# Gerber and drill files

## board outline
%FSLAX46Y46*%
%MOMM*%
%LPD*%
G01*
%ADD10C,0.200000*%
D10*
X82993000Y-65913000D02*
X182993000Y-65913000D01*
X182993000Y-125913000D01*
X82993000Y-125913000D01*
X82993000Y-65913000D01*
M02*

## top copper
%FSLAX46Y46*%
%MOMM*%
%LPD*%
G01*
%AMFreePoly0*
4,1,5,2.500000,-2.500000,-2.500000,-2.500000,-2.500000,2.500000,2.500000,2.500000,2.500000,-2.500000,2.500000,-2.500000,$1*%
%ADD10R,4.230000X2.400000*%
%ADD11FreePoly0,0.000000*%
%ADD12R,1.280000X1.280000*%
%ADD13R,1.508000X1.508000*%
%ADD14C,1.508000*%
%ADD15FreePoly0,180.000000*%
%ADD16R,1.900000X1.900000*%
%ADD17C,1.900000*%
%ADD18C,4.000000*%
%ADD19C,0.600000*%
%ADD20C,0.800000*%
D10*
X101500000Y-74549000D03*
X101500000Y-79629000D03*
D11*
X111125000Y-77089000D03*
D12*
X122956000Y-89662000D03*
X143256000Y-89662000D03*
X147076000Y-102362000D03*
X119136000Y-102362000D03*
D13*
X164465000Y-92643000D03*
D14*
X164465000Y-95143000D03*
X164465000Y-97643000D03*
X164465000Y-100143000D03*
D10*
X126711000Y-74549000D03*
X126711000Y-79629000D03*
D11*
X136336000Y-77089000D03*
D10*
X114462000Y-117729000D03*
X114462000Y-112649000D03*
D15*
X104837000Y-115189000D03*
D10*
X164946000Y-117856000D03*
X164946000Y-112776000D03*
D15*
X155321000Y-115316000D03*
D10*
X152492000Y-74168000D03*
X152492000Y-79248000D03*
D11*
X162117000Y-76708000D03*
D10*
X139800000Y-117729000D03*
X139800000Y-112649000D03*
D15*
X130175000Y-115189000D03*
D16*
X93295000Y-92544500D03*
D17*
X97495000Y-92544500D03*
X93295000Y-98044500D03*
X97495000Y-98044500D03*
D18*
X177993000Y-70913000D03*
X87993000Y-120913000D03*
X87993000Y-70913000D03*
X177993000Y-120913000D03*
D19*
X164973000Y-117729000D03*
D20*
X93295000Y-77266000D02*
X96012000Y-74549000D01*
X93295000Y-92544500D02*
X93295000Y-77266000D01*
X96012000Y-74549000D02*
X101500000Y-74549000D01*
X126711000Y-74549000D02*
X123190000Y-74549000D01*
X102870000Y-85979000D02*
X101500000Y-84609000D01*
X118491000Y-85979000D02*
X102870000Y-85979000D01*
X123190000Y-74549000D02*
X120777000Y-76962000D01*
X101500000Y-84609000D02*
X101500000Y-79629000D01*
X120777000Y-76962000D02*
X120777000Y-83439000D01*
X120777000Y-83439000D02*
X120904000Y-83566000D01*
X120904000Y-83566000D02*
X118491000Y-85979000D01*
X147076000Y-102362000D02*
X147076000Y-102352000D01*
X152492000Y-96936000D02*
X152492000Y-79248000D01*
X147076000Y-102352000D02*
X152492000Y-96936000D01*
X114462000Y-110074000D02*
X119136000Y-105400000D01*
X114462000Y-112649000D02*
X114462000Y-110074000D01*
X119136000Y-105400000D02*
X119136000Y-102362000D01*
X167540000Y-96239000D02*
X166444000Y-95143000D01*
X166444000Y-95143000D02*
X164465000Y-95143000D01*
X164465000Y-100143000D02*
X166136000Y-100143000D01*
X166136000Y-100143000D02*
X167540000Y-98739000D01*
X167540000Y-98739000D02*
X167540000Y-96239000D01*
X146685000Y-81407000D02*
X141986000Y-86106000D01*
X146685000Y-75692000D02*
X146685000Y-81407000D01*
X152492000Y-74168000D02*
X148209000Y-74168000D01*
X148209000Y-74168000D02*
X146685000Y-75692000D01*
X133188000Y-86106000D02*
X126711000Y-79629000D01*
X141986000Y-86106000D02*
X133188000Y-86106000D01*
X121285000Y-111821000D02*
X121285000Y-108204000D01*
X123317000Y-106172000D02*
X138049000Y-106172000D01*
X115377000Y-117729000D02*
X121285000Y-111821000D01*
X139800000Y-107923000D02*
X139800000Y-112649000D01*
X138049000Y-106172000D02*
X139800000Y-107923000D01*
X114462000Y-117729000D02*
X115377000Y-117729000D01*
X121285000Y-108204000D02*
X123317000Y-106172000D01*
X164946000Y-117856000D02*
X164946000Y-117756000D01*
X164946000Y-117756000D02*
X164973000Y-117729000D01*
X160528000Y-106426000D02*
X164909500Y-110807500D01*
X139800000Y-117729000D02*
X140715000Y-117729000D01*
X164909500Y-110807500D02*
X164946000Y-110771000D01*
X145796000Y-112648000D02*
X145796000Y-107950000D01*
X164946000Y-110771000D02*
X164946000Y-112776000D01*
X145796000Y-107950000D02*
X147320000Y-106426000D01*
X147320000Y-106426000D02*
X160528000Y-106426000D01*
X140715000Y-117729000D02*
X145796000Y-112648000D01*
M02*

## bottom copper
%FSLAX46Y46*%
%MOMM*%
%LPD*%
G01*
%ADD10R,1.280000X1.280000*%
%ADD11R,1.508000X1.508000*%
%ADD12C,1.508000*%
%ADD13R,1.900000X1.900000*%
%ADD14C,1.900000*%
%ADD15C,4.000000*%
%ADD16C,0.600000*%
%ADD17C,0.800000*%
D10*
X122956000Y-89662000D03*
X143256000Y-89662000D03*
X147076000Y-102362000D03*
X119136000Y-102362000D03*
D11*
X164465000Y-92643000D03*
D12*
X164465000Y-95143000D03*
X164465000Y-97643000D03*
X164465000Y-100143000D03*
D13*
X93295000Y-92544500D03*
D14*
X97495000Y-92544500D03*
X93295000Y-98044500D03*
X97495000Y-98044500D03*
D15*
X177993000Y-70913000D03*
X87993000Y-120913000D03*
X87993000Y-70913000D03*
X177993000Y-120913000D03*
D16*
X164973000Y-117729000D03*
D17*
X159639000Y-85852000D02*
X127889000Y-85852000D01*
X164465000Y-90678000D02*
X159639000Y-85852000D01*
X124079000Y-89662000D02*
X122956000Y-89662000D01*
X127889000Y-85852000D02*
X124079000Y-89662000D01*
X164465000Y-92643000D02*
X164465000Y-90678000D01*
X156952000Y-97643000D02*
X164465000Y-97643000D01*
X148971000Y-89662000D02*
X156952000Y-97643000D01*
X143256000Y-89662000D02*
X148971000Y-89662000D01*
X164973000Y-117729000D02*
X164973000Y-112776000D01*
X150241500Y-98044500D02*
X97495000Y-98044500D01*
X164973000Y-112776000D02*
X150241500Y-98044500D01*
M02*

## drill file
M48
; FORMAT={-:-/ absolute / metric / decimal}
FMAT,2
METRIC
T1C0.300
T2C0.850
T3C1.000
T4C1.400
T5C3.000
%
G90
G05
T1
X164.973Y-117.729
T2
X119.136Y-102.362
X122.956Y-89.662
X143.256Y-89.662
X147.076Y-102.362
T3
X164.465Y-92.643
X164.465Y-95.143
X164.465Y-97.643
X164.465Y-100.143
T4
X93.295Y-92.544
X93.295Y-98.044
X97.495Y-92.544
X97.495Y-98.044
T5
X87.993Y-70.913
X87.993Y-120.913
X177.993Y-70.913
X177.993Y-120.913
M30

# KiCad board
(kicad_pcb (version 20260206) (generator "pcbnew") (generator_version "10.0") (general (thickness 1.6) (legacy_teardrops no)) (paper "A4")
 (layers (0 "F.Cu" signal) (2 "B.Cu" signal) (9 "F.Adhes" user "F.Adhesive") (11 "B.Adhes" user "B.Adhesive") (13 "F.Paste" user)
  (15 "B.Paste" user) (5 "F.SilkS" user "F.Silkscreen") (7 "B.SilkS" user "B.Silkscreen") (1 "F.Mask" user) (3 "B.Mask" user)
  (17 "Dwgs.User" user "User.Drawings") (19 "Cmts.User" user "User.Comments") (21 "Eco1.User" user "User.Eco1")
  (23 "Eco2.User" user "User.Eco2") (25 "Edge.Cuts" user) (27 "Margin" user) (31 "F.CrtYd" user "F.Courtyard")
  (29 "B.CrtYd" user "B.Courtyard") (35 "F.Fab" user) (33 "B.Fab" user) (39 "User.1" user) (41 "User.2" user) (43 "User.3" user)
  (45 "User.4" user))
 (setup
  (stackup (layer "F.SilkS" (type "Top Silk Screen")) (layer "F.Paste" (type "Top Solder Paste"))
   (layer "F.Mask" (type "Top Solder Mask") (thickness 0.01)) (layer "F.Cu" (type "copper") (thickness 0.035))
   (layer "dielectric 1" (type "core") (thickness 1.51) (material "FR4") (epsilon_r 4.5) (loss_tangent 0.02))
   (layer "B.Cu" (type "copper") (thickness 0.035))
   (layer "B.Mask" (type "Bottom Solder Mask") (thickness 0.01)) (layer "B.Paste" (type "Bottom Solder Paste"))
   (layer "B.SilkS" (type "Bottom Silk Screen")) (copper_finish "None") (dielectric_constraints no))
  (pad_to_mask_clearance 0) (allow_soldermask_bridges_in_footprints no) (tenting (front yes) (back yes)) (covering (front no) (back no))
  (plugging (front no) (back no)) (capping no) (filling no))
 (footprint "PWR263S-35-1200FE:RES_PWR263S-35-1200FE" (layer "F.Cu") (at 107.885 77.089)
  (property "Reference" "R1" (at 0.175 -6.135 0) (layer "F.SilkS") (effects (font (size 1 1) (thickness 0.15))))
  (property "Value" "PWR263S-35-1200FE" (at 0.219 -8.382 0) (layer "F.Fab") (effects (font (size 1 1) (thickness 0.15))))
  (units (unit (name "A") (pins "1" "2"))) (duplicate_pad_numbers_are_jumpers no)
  (pad "1" smd rect (at -6.385 -2.54) (size 4.23 2.4) (layers "F.Cu" "F.Mask" "F.Paste") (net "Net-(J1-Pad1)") (solder_mask_margin 0.102))
  (pad "2" smd rect (at -6.385 2.54) (size 4.23 2.4) (layers "F.Cu" "F.Mask" "F.Paste") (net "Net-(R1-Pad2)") (solder_mask_margin 0.102))
  (pad "3" smd custom (at 3.24 0) (size 5 5) (layers "F.Cu") (options (clearance outline) (anchor rect)) (primitives)))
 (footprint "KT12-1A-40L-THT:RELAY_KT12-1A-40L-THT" (layer "F.Cu") (at 133.106 96.012)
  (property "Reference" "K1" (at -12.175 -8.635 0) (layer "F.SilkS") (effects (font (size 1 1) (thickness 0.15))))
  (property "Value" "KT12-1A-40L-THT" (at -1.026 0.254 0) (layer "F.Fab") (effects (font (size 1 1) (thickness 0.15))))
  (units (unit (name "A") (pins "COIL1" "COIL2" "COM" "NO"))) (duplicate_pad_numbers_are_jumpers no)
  (pad "COIL1" thru_hole rect (at -10.15 -6.35) (size 1.28 1.28) (drill 0.85) (layers "*.Cu" "*.Mask") (remove_unused_layers no)
   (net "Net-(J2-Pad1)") (solder_mask_margin 0.102))
  (pad "COIL2" thru_hole rect (at 10.15 -6.35) (size 1.28 1.28) (drill 0.85) (layers "*.Cu" "*.Mask") (remove_unused_layers no)
   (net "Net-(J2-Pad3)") (solder_mask_margin 0.102))
  (pad "COM" thru_hole rect (at 13.97 6.35) (size 1.28 1.28) (drill 0.85) (layers "*.Cu" "*.Mask") (remove_unused_layers no)
   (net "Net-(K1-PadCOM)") (solder_mask_margin 0.102))
  (pad "NO" thru_hole rect (at -13.97 6.35) (size 1.28 1.28) (drill 0.85) (layers "*.Cu" "*.Mask") (remove_unused_layers no)
   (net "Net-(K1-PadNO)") (solder_mask_margin 0.102)))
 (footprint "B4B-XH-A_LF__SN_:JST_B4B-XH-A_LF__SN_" (layer "F.Cu") (at 163.94 96.393 90)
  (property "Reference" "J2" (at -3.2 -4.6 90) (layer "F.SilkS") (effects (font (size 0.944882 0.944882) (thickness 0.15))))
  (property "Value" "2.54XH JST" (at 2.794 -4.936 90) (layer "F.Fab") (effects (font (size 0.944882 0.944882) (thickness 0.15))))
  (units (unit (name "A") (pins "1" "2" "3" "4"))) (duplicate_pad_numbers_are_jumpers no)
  (pad "1" thru_hole rect (at 3.75 0.525 90) (size 1.508 1.508) (drill 1) (layers "*.Cu" "*.Mask") (remove_unused_layers no)
   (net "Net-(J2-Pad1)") (solder_mask_margin 0.102))
  (pad "2" thru_hole circle (at 1.25 0.525 90) (size 1.508 1.508) (drill 1) (layers "*.Cu" "*.Mask") (remove_unused_layers no) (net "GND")
   (solder_mask_margin 0.102))
  (pad "3" thru_hole circle (at -1.25 0.525 90) (size 1.508 1.508) (drill 1) (layers "*.Cu" "*.Mask") (remove_unused_layers no)
   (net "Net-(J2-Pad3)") (solder_mask_margin 0.102))
  (pad "4" thru_hole circle (at -3.75 0.525 90) (size 1.508 1.508) (drill 1) (layers "*.Cu" "*.Mask") (remove_unused_layers no) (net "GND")
   (solder_mask_margin 0.102)))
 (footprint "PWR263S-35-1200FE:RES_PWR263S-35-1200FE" (layer "F.Cu") (at 133.096 77.089)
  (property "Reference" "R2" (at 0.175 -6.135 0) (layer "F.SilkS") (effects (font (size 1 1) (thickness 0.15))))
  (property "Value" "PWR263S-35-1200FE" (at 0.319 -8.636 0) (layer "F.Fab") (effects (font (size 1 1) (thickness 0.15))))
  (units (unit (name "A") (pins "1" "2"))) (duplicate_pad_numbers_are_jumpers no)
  (pad "1" smd rect (at -6.385 -2.54) (size 4.23 2.4) (layers "F.Cu" "F.Mask" "F.Paste") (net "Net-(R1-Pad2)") (solder_mask_margin 0.102))
  (pad "2" smd rect (at -6.385 2.54) (size 4.23 2.4) (layers "F.Cu" "F.Mask" "F.Paste") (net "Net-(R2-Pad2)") (solder_mask_margin 0.102))
  (pad "3" smd custom (at 3.24 0) (size 5 5) (layers "F.Cu") (options (clearance outline) (anchor rect)) (primitives)))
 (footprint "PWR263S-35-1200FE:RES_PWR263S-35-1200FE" (layer "F.Cu") (at 108.077 115.189 180)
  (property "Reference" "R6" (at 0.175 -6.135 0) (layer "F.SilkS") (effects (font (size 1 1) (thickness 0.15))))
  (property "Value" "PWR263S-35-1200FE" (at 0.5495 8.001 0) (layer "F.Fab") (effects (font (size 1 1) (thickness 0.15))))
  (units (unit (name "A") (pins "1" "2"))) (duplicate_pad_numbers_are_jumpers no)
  (pad "1" smd rect (at -6.385 -2.54 180) (size 4.23 2.4) (layers "F.Cu" "F.Mask" "F.Paste") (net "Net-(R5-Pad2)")
   (solder_mask_margin 0.102))
  (pad "2" smd rect (at -6.385 2.54 180) (size 4.23 2.4) (layers "F.Cu" "F.Mask" "F.Paste") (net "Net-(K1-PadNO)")
   (solder_mask_margin 0.102))
  (pad "3" smd custom (at 3.24 0 180) (size 5 5) (layers "F.Cu") (options (clearance outline) (anchor rect)) (primitives)))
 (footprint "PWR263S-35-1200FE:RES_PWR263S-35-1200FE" (layer "F.Cu") (at 158.561 115.316 180)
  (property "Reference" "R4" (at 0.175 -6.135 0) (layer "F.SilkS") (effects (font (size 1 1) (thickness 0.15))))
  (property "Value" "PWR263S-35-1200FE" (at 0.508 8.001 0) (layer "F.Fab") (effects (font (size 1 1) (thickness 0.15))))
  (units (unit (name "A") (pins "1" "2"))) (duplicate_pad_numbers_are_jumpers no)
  (pad "1" smd rect (at -6.385 -2.54 180) (size 4.23 2.4) (layers "F.Cu" "F.Mask" "F.Paste") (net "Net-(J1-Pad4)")
   (solder_mask_margin 0.102))
  (pad "2" smd rect (at -6.385 2.54 180) (size 4.23 2.4) (layers "F.Cu" "F.Mask" "F.Paste") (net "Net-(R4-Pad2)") (solder_mask_margin 0.102))
  (pad "3" smd custom (at 3.24 0 180) (size 5 5) (layers "F.Cu") (options (clearance outline) (anchor rect)) (primitives)))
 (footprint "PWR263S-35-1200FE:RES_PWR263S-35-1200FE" (layer "F.Cu") (at 158.877 76.708)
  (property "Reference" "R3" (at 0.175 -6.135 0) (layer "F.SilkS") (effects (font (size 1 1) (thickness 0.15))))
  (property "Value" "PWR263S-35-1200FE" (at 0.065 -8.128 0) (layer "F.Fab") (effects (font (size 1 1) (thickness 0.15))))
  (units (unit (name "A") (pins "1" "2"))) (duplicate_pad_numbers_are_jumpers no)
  (pad "1" smd rect (at -6.385 -2.54) (size 4.23 2.4) (layers "F.Cu" "F.Mask" "F.Paste") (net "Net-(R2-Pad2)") (solder_mask_margin 0.102))
  (pad "2" smd rect (at -6.385 2.54) (size 4.23 2.4) (layers "F.Cu" "F.Mask" "F.Paste") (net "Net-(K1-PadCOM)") (solder_mask_margin 0.102))
  (pad "3" smd custom (at 3.24 0) (size 5 5) (layers "F.Cu") (options (clearance outline) (anchor rect)) (primitives)))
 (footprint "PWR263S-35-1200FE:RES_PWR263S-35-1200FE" (layer "F.Cu") (at 133.415 115.189 180)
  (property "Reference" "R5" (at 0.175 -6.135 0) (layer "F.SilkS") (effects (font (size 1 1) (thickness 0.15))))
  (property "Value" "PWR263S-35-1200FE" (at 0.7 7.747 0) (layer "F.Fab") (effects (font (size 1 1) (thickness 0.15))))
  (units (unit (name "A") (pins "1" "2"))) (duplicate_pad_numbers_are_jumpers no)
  (pad "1" smd rect (at -6.385 -2.54 180) (size 4.23 2.4) (layers "F.Cu" "F.Mask" "F.Paste") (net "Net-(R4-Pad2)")
   (solder_mask_margin 0.102))
  (pad "2" smd rect (at -6.385 2.54 180) (size 4.23 2.4) (layers "F.Cu" "F.Mask" "F.Paste") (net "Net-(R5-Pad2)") (solder_mask_margin 0.102))
  (pad "3" smd custom (at 3.24 0 180) (size 5 5) (layers "F.Cu") (options (clearance outline) (anchor rect)) (primitives)))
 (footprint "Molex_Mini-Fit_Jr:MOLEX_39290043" (layer "F.Cu") (at 93.295 92.5445)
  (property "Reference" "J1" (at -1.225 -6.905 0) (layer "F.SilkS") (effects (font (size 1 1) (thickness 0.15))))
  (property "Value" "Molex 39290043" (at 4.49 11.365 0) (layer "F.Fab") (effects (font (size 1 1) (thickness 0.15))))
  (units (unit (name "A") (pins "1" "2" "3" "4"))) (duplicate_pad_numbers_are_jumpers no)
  (pad "1" thru_hole rect (at 0 0) (size 1.9 1.9) (drill 1.4) (layers "*.Cu") (remove_unused_layers no) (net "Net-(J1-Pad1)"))
  (pad "2" thru_hole circle (at 4.2 0) (size 1.9 1.9) (drill 1.4) (layers "*.Cu") (remove_unused_layers no) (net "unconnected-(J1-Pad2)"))
  (pad "3" thru_hole circle (at 0 5.5) (size 1.9 1.9) (drill 1.4) (layers "*.Cu") (remove_unused_layers no) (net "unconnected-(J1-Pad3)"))
  (pad "4" thru_hole circle (at 4.2 5.5) (size 1.9 1.9) (drill 1.4) (layers "*.Cu") (remove_unused_layers no) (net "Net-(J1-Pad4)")))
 (gr_rect (start 82.993 65.913) (end 182.993 125.913) (stroke (width 0.2) (type solid)) (fill no) (layer "Edge.Cuts"))
 (via (at 177.993 70.913) (size 4) (drill 3) (layers "F.Cu" "B.Cu") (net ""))
 (via (at 87.993 120.913) (size 4) (drill 3) (layers "F.Cu" "B.Cu") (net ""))
 (via (at 87.993 70.913) (size 4) (drill 3) (layers "F.Cu" "B.Cu") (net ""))
 (via (at 177.993 120.913) (size 4) (drill 3) (layers "F.Cu" "B.Cu") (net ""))
 (segment (start 93.295 77.266) (end 96.012 74.549) (width 0.8) (layer "F.Cu") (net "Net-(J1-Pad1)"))
 (segment (start 93.295 92.5445) (end 93.295 77.266) (width 0.8) (layer "F.Cu") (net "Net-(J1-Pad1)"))
 (segment (start 96.012 74.549) (end 101.5 74.549) (width 0.8) (layer "F.Cu") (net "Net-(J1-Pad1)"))
 (segment (start 126.711 74.549) (end 123.19 74.549) (width 0.8) (layer "F.Cu") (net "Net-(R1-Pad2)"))
 (segment (start 102.87 85.979) (end 101.5 84.609) (width 0.8) (layer "F.Cu") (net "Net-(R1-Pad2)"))
 (segment (start 118.491 85.979) (end 102.87 85.979) (width 0.8) (layer "F.Cu") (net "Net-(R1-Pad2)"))
 (segment (start 123.19 74.549) (end 120.777 76.962) (width 0.8) (layer "F.Cu") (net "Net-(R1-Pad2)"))
 (segment (start 101.5 84.609) (end 101.5 79.629) (width 0.8) (layer "F.Cu") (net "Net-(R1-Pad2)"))
 (segment (start 120.777 76.962) (end 120.777 83.439) (width 0.8) (layer "F.Cu") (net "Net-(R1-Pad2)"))
 (segment (start 120.777 83.439) (end 120.904 83.566) (width 0.8) (layer "F.Cu") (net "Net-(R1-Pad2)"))
 (segment (start 120.904 83.566) (end 118.491 85.979) (width 0.8) (layer "F.Cu") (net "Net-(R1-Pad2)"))
 (segment (start 159.639 85.852) (end 127.889 85.852) (width 0.8) (layer "B.Cu") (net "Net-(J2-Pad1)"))
 (segment (start 164.465 90.678) (end 159.639 85.852) (width 0.8) (layer "B.Cu") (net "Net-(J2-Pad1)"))
 (segment (start 124.079 89.662) (end 122.956 89.662) (width 0.8) (layer "B.Cu") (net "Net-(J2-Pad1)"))
 (segment (start 127.889 85.852) (end 124.079 89.662) (width 0.8) (layer "B.Cu") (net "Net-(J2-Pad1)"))
 (segment (start 164.465 92.643) (end 164.465 90.678) (width 0.8) (layer "B.Cu") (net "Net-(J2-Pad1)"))
 (segment (start 156.952 97.643) (end 164.465 97.643) (width 0.8) (layer "B.Cu") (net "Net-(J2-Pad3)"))
 (segment (start 148.971 89.662) (end 156.952 97.643) (width 0.8) (layer "B.Cu") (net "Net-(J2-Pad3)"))
 (segment (start 143.256 89.662) (end 148.971 89.662) (width 0.8) (layer "B.Cu") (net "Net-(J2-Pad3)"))
 (segment (start 147.076 102.362) (end 147.076 102.352) (width 0.8) (layer "F.Cu") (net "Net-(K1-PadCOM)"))
 (segment (start 152.492 96.936) (end 152.492 79.248) (width 0.8) (layer "F.Cu") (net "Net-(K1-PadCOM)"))
 (segment (start 147.076 102.352) (end 152.492 96.936) (width 0.8) (layer "F.Cu") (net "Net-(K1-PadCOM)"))
 (segment (start 114.462 110.074) (end 119.136 105.4) (width 0.8) (layer "F.Cu") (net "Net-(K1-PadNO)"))
 (segment (start 114.462 112.649) (end 114.462 110.074) (width 0.8) (layer "F.Cu") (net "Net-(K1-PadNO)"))
 (segment (start 119.136 105.4) (end 119.136 102.362) (width 0.8) (layer "F.Cu") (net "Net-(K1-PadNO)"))
 (segment (start 167.54 96.239) (end 166.444 95.143) (width 0.8) (layer "F.Cu") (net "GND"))
 (segment (start 166.444 95.143) (end 164.465 95.143) (width 0.8) (layer "F.Cu") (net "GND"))
 (segment (start 164.465 100.143) (end 166.136 100.143) (width 0.8) (layer "F.Cu") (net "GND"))
 (segment (start 166.136 100.143) (end 167.54 98.739) (width 0.8) (layer "F.Cu") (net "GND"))
 (segment (start 167.54 98.739) (end 167.54 96.239) (width 0.8) (layer "F.Cu") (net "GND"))
 (segment (start 146.685 81.407) (end 141.986 86.106) (width 0.8) (layer "F.Cu") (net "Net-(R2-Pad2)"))
 (segment (start 146.685 75.692) (end 146.685 81.407) (width 0.8) (layer "F.Cu") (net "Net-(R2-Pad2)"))
 (segment (start 152.492 74.168) (end 148.209 74.168) (width 0.8) (layer "F.Cu") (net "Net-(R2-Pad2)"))
 (segment (start 148.209 74.168) (end 146.685 75.692) (width 0.8) (layer "F.Cu") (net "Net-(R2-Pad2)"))
 (segment (start 133.188 86.106) (end 126.711 79.629) (width 0.8) (layer "F.Cu") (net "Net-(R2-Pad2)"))
 (segment (start 141.986 86.106) (end 133.188 86.106) (width 0.8) (layer "F.Cu") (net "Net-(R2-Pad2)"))
 (segment (start 121.285 111.821) (end 121.285 108.204) (width 0.8) (layer "F.Cu") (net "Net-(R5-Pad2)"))
 (segment (start 123.317 106.172) (end 138.049 106.172) (width 0.8) (layer "F.Cu") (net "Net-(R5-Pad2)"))
 (segment (start 115.377 117.729) (end 121.285 111.821) (width 0.8) (layer "F.Cu") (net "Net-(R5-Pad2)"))
 (segment (start 139.8 107.923) (end 139.8 112.649) (width 0.8) (layer "F.Cu") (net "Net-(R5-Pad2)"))
 (segment (start 138.049 106.172) (end 139.8 107.923) (width 0.8) (layer "F.Cu") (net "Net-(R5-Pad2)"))
 (segment (start 114.462 117.729) (end 115.377 117.729) (width 0.8) (layer "F.Cu") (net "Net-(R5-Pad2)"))
 (segment (start 121.285 108.204) (end 123.317 106.172) (width 0.8) (layer "F.Cu") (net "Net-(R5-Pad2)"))
 (segment (start 164.946 117.856) (end 164.946 117.756) (width 0.8) (layer "F.Cu") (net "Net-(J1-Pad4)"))
 (segment (start 164.946 117.756) (end 164.973 117.729) (width 0.8) (layer "F.Cu") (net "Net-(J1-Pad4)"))
 (via (at 164.973 117.729) (size 0.6) (drill 0.3) (layers "F.Cu" "B.Cu") (free yes) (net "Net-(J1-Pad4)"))
 (segment (start 164.973 117.729) (end 164.973 112.776) (width 0.8) (layer "B.Cu") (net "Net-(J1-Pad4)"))
 (segment (start 150.2415 98.0445) (end 97.495 98.0445) (width 0.8) (layer "B.Cu") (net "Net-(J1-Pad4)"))
 (segment (start 164.973 112.776) (end 150.2415 98.0445) (width 0.8) (layer "B.Cu") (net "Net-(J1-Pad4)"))
 (segment (start 160.528 106.426) (end 164.9095 110.8075) (width 0.8) (layer "F.Cu") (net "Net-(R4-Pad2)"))
 (segment (start 139.8 117.729) (end 140.715 117.729) (width 0.8) (layer "F.Cu") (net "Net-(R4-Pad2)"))
 (segment (start 164.9095 110.8075) (end 164.946 110.771) (width 0.8) (layer "F.Cu") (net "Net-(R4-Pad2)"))
 (segment (start 145.796 112.648) (end 145.796 107.95) (width 0.8) (layer "F.Cu") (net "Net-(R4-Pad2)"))
 (segment (start 164.946 110.771) (end 164.946 112.776) (width 0.8) (layer "F.Cu") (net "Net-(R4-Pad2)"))
 (segment (start 145.796 107.95) (end 147.32 106.426) (width 0.8) (layer "F.Cu") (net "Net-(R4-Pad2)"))
 (segment (start 147.32 106.426) (end 160.528 106.426) (width 0.8) (layer "F.Cu") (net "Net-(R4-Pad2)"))
 (segment (start 140.715 117.729) (end 145.796 112.648) (width 0.8) (layer "F.Cu") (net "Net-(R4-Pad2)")))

